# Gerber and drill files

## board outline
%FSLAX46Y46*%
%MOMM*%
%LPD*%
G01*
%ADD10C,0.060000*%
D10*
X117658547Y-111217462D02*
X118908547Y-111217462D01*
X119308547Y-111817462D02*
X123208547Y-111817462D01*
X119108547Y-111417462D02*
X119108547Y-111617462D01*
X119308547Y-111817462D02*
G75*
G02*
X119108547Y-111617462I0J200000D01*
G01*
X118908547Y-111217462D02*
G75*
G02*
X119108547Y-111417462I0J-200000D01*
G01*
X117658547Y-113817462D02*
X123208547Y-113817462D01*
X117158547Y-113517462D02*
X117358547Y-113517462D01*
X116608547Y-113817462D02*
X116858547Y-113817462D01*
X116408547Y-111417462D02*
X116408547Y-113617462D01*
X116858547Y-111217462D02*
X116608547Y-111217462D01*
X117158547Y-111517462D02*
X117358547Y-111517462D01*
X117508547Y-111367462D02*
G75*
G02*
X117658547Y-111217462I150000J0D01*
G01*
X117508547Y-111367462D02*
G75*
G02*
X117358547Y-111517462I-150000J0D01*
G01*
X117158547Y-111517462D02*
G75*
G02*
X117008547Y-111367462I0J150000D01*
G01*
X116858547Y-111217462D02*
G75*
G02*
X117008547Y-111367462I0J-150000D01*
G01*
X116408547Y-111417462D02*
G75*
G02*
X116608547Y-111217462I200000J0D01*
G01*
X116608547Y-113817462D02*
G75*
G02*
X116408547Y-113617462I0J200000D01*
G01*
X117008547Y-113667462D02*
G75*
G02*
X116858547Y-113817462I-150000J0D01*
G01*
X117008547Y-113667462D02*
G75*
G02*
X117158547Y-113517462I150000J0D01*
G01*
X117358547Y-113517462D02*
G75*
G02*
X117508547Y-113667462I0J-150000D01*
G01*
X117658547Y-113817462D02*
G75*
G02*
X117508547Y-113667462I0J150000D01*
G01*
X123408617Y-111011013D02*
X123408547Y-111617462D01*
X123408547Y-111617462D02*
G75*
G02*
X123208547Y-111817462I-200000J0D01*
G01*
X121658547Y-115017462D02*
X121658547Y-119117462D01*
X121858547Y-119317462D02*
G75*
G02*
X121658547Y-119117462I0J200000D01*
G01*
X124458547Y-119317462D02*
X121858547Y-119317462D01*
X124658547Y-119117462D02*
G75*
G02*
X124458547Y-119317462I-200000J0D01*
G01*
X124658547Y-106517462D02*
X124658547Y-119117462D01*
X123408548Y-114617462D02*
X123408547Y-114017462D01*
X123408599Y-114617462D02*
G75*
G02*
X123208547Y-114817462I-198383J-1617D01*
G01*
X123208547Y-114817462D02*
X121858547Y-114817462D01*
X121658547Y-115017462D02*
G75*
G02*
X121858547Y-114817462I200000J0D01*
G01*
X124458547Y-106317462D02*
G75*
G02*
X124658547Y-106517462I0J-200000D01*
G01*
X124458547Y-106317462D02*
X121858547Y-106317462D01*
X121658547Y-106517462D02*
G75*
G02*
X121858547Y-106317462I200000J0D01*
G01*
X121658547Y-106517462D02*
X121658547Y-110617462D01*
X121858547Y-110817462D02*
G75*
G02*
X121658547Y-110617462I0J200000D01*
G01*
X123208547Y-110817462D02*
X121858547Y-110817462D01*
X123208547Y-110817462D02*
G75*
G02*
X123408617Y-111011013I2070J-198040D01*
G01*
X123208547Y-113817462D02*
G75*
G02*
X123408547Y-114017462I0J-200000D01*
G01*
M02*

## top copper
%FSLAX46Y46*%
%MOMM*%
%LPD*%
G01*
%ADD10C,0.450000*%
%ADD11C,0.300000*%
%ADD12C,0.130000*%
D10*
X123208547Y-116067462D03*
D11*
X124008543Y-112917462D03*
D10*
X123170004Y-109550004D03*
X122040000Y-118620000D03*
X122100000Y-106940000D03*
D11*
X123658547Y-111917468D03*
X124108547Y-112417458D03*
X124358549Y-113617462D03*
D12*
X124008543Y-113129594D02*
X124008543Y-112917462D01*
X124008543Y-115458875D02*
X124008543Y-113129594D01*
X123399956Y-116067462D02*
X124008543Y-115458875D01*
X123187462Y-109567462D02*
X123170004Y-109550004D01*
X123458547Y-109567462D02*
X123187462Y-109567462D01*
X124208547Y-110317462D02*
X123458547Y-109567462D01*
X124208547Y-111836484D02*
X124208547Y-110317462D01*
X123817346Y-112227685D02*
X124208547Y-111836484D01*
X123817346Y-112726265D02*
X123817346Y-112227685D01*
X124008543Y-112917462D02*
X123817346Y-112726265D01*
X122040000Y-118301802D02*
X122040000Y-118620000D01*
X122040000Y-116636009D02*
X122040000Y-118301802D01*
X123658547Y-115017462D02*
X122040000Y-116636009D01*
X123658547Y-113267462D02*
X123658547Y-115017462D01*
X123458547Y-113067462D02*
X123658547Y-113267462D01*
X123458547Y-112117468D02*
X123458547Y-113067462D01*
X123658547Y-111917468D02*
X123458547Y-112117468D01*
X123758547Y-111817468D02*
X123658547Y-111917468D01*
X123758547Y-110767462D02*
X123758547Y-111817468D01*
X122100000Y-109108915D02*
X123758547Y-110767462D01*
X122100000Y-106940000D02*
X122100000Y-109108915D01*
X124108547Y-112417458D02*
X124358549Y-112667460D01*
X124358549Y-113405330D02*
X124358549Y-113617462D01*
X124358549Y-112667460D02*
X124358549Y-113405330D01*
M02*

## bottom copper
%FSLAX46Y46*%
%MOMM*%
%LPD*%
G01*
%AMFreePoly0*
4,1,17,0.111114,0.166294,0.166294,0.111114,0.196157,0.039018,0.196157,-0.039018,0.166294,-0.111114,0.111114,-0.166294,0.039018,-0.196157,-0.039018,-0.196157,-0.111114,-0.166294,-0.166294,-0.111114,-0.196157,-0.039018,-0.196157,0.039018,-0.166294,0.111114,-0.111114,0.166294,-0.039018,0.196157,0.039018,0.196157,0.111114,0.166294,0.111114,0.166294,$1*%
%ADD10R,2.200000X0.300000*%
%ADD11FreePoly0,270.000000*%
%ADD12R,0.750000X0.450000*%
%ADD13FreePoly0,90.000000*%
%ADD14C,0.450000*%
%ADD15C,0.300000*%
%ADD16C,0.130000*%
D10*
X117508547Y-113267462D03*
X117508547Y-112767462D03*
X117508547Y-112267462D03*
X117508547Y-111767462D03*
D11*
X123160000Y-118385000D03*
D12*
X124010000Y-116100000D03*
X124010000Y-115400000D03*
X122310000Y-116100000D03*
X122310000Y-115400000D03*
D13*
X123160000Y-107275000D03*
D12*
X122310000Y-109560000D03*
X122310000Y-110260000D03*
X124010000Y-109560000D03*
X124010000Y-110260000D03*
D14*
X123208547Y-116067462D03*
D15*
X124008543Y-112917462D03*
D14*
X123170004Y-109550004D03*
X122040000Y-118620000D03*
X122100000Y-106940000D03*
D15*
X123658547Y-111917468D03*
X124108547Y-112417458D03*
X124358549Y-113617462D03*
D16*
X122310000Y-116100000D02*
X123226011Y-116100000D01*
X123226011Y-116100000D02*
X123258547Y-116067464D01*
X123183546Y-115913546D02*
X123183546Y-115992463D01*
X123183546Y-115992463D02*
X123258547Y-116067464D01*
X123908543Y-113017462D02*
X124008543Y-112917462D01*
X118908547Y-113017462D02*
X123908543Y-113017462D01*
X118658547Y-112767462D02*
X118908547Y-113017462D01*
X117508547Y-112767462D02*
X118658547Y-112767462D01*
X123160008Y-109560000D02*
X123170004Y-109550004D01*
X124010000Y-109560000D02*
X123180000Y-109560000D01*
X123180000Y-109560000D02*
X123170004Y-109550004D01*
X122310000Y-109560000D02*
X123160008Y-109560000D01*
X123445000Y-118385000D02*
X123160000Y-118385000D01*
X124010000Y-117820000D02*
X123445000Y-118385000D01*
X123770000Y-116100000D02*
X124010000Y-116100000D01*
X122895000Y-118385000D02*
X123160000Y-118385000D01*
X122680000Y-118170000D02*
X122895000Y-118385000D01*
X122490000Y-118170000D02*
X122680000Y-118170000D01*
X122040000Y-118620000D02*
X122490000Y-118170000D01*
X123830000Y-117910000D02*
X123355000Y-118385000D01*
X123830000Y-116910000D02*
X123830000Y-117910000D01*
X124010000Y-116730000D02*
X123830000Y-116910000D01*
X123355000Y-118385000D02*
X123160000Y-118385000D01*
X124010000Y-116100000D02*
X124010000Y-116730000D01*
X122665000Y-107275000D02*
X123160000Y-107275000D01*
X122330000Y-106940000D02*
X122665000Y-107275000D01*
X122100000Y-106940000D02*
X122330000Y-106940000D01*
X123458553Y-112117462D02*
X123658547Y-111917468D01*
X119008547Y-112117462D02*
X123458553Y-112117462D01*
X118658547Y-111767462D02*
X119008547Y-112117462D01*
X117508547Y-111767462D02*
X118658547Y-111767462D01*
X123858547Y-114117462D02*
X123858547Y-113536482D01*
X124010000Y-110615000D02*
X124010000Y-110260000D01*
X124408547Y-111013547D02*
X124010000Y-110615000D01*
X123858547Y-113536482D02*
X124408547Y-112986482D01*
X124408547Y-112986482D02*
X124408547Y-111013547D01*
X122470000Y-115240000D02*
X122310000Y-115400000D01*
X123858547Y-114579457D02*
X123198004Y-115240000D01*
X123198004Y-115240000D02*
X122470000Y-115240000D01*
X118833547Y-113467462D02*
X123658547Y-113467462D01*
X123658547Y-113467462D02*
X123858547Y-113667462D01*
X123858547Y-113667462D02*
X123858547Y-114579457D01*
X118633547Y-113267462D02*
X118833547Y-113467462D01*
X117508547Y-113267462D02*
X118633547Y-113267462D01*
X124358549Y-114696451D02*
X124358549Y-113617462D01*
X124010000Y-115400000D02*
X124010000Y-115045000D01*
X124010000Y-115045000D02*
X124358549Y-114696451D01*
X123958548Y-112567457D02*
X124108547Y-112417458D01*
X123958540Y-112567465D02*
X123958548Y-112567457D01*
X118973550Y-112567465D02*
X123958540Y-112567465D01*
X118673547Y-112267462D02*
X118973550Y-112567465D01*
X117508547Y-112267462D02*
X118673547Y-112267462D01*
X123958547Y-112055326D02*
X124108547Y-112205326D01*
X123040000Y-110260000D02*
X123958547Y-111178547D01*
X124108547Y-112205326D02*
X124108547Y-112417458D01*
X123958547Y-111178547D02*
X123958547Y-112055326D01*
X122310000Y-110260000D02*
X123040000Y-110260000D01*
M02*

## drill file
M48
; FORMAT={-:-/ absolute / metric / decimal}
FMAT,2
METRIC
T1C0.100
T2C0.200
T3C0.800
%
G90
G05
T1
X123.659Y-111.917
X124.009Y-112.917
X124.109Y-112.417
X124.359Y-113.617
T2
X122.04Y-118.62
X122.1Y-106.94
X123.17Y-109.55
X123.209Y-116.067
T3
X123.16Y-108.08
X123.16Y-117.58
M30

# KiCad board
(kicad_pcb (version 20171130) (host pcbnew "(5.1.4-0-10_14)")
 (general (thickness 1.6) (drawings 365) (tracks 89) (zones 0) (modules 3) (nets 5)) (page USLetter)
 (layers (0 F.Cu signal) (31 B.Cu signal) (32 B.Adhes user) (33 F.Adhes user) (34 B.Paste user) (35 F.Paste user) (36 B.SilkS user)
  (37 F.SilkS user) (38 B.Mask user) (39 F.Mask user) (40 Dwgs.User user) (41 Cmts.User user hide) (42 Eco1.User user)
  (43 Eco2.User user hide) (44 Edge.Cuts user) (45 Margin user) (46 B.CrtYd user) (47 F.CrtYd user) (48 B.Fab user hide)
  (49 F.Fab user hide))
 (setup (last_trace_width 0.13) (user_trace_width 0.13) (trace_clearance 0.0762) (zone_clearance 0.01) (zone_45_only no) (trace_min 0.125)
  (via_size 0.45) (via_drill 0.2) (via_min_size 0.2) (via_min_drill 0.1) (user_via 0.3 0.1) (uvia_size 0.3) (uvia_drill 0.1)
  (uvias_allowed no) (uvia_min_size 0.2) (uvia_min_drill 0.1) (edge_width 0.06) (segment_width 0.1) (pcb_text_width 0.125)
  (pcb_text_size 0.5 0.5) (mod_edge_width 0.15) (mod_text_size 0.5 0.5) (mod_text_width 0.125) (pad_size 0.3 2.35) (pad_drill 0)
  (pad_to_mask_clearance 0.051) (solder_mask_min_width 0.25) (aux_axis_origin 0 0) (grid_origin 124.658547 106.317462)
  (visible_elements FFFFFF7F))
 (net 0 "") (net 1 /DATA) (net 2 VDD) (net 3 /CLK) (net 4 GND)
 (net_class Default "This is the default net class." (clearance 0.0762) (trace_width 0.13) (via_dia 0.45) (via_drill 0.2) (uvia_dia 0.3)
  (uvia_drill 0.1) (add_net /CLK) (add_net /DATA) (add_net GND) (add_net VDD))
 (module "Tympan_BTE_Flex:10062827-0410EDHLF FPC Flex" (layer B.Cu) (at 116.408547 111.217462 270)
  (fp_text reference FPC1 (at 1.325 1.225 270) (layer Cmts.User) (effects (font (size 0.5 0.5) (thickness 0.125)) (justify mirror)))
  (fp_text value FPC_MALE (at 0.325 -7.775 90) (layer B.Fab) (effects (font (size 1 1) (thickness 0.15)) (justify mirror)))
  (pad 1 smd rect (at 2.05 -1.1 270) (size 0.3 2.2) (layers B.Cu B.Mask) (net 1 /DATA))
  (pad 2 smd rect (at 1.55 -1.1 270) (size 0.3 2.2) (layers B.Cu B.Mask) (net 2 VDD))
  (pad 3 smd rect (at 1.05 -1.1 270) (size 0.3 2.2) (layers B.Cu B.Mask) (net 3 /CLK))
  (pad 4 smd rect (at 0.55 -1.1 270) (size 0.3 2.2) (layers B.Cu B.Mask) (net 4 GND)))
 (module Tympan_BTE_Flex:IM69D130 (layer B.Cu) (at 123.16 117.58 270)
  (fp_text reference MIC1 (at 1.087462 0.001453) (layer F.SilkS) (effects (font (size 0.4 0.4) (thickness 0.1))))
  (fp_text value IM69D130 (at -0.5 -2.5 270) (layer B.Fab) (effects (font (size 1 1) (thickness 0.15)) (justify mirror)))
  (pad "" np_thru_hole circle (at 0 0 270) (size 0.8 0.8) (drill 0.8) (layers *.Cu *.Mask))
  (pad 5 smd custom (at 0.805 0 270) (size 0.4 0.4) (layers B.Cu B.Mask) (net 4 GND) (zone_connect 0)
   (options (clearance outline) (anchor circle)) (primitives))
  (pad 4 smd rect (at -1.48 -0.85 270) (size 0.45 0.75) (layers B.Cu B.Mask) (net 4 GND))
  (pad 3 smd rect (at -2.18 -0.85 270) (size 0.45 0.75) (layers B.Cu B.Mask) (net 3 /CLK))
  (pad 2 smd rect (at -1.48 0.85 270) (size 0.45 0.75) (layers B.Cu B.Mask) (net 2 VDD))
  (pad 1 smd rect (at -2.18 0.85 270) (size 0.45 0.75) (layers B.Cu B.Mask) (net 1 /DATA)))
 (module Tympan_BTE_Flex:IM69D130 (layer B.Cu) (at 123.16 108.76 90)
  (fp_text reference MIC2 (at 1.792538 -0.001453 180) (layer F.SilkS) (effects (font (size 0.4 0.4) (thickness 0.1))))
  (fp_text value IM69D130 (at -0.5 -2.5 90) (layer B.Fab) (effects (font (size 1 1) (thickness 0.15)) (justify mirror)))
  (pad "" np_thru_hole circle (at 0.68 0 90) (size 0.8 0.8) (drill 0.8) (layers *.Cu *.Mask))
  (pad 5 smd custom (at 1.485 0 90) (size 0.4 0.4) (layers B.Cu B.Mask) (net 4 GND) (zone_connect 0)
   (options (clearance outline) (anchor circle)) (primitives))
  (pad 4 smd rect (at -0.8 -0.85 90) (size 0.45 0.75) (layers B.Cu B.Mask) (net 2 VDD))
  (pad 3 smd rect (at -1.5 -0.85 90) (size 0.45 0.75) (layers B.Cu B.Mask) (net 3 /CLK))
  (pad 2 smd rect (at -0.8 0.85 90) (size 0.45 0.75) (layers B.Cu B.Mask) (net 2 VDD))
  (pad 1 smd rect (at -1.5 0.85 90) (size 0.45 0.75) (layers B.Cu B.Mask) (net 1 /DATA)))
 (gr_line (start 117.658547 111.217462) (end 118.908547 111.217462) (layer Edge.Cuts) (width 0.06))
 (gr_line (start 119.308547 111.817462) (end 123.208547 111.817462) (layer Edge.Cuts) (width 0.06))
 (gr_line (start 119.108547 111.417462) (end 119.108547 111.617462) (layer Edge.Cuts) (width 0.06))
 (gr_arc (start 119.308547 111.617462) (end 119.108547 111.617462) (angle -90) (layer Edge.Cuts) (width 0.06))
 (gr_arc (start 118.908547 111.417462) (end 119.108547 111.417462) (angle -90) (layer Edge.Cuts) (width 0.06))
 (gr_line (start 117.658547 113.817462) (end 123.208547 113.817462) (layer Edge.Cuts) (width 0.06))
 (gr_line (start 117.158547 113.517462) (end 117.358547 113.517462) (layer Edge.Cuts) (width 0.06))
 (gr_line (start 116.608547 113.817462) (end 116.858547 113.817462) (layer Edge.Cuts) (width 0.06))
 (gr_line (start 116.408547 111.417462) (end 116.408547 113.617462) (layer Edge.Cuts) (width 0.06))
 (gr_line (start 116.858547 111.217462) (end 116.608547 111.217462) (layer Edge.Cuts) (width 0.06))
 (gr_line (start 117.158547 111.517462) (end 117.358547 111.517462) (layer Edge.Cuts) (width 0.06))
 (gr_arc (start 117.658547 111.367462) (end 117.658547 111.217462) (angle -90) (layer Edge.Cuts) (width 0.06))
 (gr_arc (start 117.358547 111.367462) (end 117.358547 111.517462) (angle -90) (layer Edge.Cuts) (width 0.06))
 (gr_arc (start 117.158547 111.367462) (end 117.008547 111.367462) (angle -90) (layer Edge.Cuts) (width 0.06))
 (gr_arc (start 116.858547 111.367462) (end 117.008547 111.367462) (angle -90) (layer Edge.Cuts) (width 0.06))
 (gr_arc (start 116.608547 111.417462) (end 116.608547 111.217462) (angle -90) (layer Edge.Cuts) (width 0.06))
 (gr_arc (start 116.608547 113.617462) (end 116.408547 113.617462) (angle -90) (layer Edge.Cuts) (width 0.06))
 (gr_arc (start 116.858547 113.667462) (end 116.858547 113.817462) (angle -90) (layer Edge.Cuts) (width 0.06))
 (gr_arc (start 117.158547 113.667462) (end 117.158547 113.517462) (angle -90) (layer Edge.Cuts) (width 0.06))
 (gr_arc (start 117.358547 113.667462) (end 117.508547 113.667462) (angle -90) (layer Edge.Cuts) (width 0.06))
 (gr_arc (start 117.658547 113.667462) (end 117.508547 113.667462) (angle -90) (layer Edge.Cuts) (width 0.06))
 (gr_line (start 123.408617 111.011013) (end 123.408547 111.617462) (layer Edge.Cuts) (width 0.06))
 (gr_arc (start 123.208547 111.617462) (end 123.208547 111.817462) (angle -90) (layer Edge.Cuts) (width 0.06))
 (gr_line (start 121.658547 115.017462) (end 121.658547 119.117462) (layer Edge.Cuts) (width 0.06))
 (gr_arc (start 121.858547 119.117462) (end 121.658547 119.117462) (angle -90) (layer Edge.Cuts) (width 0.06))
 (gr_line (start 124.458547 119.317462) (end 121.858547 119.317462) (layer Edge.Cuts) (width 0.06))
 (gr_arc (start 124.458547 119.117462) (end 124.458547 119.317462) (angle -90) (layer Edge.Cuts) (width 0.06))
 (gr_line (start 124.658547 106.517462) (end 124.658547 119.117462) (layer Edge.Cuts) (width 0.06))
 (gr_line (start 123.408548 114.617462) (end 123.408547 114.017462) (layer Edge.Cuts) (width 0.06))
 (gr_arc (start 123.210216 114.619079) (end 123.208547 114.817462) (angle -90.94914104) (layer Edge.Cuts) (width 0.06))
 (gr_line (start 123.208547 114.817462) (end 121.858547 114.817462) (layer Edge.Cuts) (width 0.06))
 (gr_arc (start 121.858547 115.017462) (end 121.858547 114.817462) (angle -90) (layer Edge.Cuts) (width 0.06))
 (gr_arc (start 124.458547 106.517462) (end 124.658547 106.517462) (angle -90) (layer Edge.Cuts) (width 0.06))
 (gr_line (start 124.458547 106.317462) (end 121.858547 106.317462) (layer Edge.Cuts) (width 0.06))
 (gr_arc (start 121.858547 106.517462) (end 121.858547 106.317462) (angle -90) (layer Edge.Cuts) (width 0.06))
 (gr_line (start 121.658547 106.517462) (end 121.658547 110.617462) (layer Edge.Cuts) (width 0.06))
 (gr_arc (start 121.858547 110.617462) (end 121.658547 110.617462) (angle -90) (layer Edge.Cuts) (width 0.06))
 (gr_line (start 123.208547 110.817462) (end 121.858547 110.817462) (layer Edge.Cuts) (width 0.06))
 (gr_arc (start 123.210617 111.015502) (end 123.408617 111.011013) (angle -89.3) (layer Edge.Cuts) (width 0.06))
 (gr_arc (start 123.208547 114.017462) (end 123.408547 114.017462) (angle -90) (layer Edge.Cuts) (width 0.06))
 (via (at 123.208547 116.067462) (size 0.45) (drill 0.2) (layers F.Cu B.Cu) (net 2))
 (segment (start 122.31 116.1) (end 123.226011 116.1) (width 0.13) (layer B.Cu) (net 2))
 (segment (start 123.226011 116.1) (end 123.258547 116.067464) (width 0.13) (layer B.Cu) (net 2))
 (segment (start 123.183546 115.913546) (end 123.183546 115.992463) (width 0.13) (layer B.Cu) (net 2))
 (segment (start 123.183546 115.992463) (end 123.258547 116.067464) (width 0.13) (layer B.Cu) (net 2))
 (via (at 124.008543 112.917462) (size 0.3) (drill 0.1) (layers F.Cu B.Cu) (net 2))
 (segment (start 124.008543 113.129594) (end 124.008543 112.917462) (width 0.13) (layer F.Cu) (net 2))
 (segment (start 124.008543 115.458875) (end 124.008543 113.129594) (width 0.13) (layer F.Cu) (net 2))
 (segment (start 123.399956 116.067462) (end 124.008543 115.458875) (width 0.13) (layer F.Cu) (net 2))
 (segment (start 123.908543 113.017462) (end 124.008543 112.917462) (width 0.13) (layer B.Cu) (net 2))
 (segment (start 118.908547 113.017462) (end 123.908543 113.017462) (width 0.13) (layer B.Cu) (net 2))
 (segment (start 118.658547 112.767462) (end 118.908547 113.017462) (width 0.13) (layer B.Cu) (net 2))
 (segment (start 117.508547 112.767462) (end 118.658547 112.767462) (width 0.13) (layer B.Cu) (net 2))
 (via (at 123.170004 109.550004) (size 0.45) (drill 0.2) (layers F.Cu B.Cu) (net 2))
 (segment (start 123.160008 109.56) (end 123.170004 109.550004) (width 0.13) (layer B.Cu) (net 2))
 (segment (start 124.01 109.56) (end 123.18 109.56) (width 0.13) (layer B.Cu) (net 2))
 (segment (start 123.18 109.56) (end 123.170004 109.550004) (width 0.13) (layer B.Cu) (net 2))
 (segment (start 122.31 109.56) (end 123.160008 109.56) (width 0.13) (layer B.Cu) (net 2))
 (segment (start 123.187462 109.567462) (end 123.170004 109.550004) (width 0.13) (layer F.Cu) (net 2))
 (segment (start 123.458547 109.567462) (end 123.187462 109.567462) (width 0.13) (layer F.Cu) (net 2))
 (segment (start 124.208547 110.317462) (end 123.458547 109.567462) (width 0.13) (layer F.Cu) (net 2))
 (segment (start 124.208547 111.836484) (end 124.208547 110.317462) (width 0.13) (layer F.Cu) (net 2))
 (segment (start 123.817346 112.227685) (end 124.208547 111.836484) (width 0.13) (layer F.Cu) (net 2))
 (segment (start 123.817346 112.726265) (end 123.817346 112.227685) (width 0.13) (layer F.Cu) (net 2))
 (segment (start 124.008543 112.917462) (end 123.817346 112.726265) (width 0.13) (layer F.Cu) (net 2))
 (segment (start 123.445 118.385) (end 123.16 118.385) (width 0.13) (layer B.Cu) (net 4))
 (segment (start 124.01 117.82) (end 123.445 118.385) (width 0.13) (layer B.Cu) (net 4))
 (segment (start 123.77 116.1) (end 124.01 116.1) (width 0.13) (layer B.Cu) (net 4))
 (via (at 122.04 118.62) (size 0.45) (drill 0.2) (layers F.Cu B.Cu) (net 4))
 (segment (start 122.895 118.385) (end 123.16 118.385) (width 0.13) (layer B.Cu) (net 4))
 (segment (start 122.68 118.17) (end 122.895 118.385) (width 0.13) (layer B.Cu) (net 4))
 (segment (start 122.49 118.17) (end 122.68 118.17) (width 0.13) (layer B.Cu) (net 4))
 (segment (start 122.04 118.62) (end 122.49 118.17) (width 0.13) (layer B.Cu) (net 4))
 (segment (start 123.83 117.91) (end 123.355 118.385) (width 0.13) (layer B.Cu) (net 4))
 (segment (start 123.83 116.91) (end 123.83 117.91) (width 0.13) (layer B.Cu) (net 4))
 (segment (start 124.01 116.73) (end 123.83 116.91) (width 0.13) (layer B.Cu) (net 4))
 (segment (start 123.355 118.385) (end 123.16 118.385) (width 0.13) (layer B.Cu) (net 4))
 (segment (start 124.01 116.1) (end 124.01 116.73) (width 0.13) (layer B.Cu) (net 4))
 (via (at 122.1 106.94) (size 0.45) (drill 0.2) (layers F.Cu B.Cu) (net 4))
 (segment (start 122.665 107.275) (end 123.16 107.275) (width 0.13) (layer B.Cu) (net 4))
 (segment (start 122.33 106.94) (end 122.665 107.275) (width 0.13) (layer B.Cu) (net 4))
 (segment (start 122.1 106.94) (end 122.33 106.94) (width 0.13) (layer B.Cu) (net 4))
 (via (at 123.658547 111.917468) (size 0.3) (drill 0.1) (layers F.Cu B.Cu) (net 4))
 (segment (start 123.458553 112.117462) (end 123.658547 111.917468) (width 0.13) (layer B.Cu) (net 4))
 (segment (start 119.008547 112.117462) (end 123.458553 112.117462) (width 0.13) (layer B.Cu) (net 4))
 (segment (start 118.658547 111.767462) (end 119.008547 112.117462) (width 0.13) (layer B.Cu) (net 4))
 (segment (start 117.508547 111.767462) (end 118.658547 111.767462) (width 0.13) (layer B.Cu) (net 4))
 (segment (start 122.04 118.301802) (end 122.04 118.62) (width 0.13) (layer F.Cu) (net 4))
 (segment (start 122.04 116.636009) (end 122.04 118.301802) (width 0.13) (layer F.Cu) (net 4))
 (segment (start 123.658547 115.017462) (end 122.04 116.636009) (width 0.13) (layer F.Cu) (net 4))
 (segment (start 123.658547 113.267462) (end 123.658547 115.017462) (width 0.13) (layer F.Cu) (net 4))
 (segment (start 123.458547 113.067462) (end 123.658547 113.267462) (width 0.13) (layer F.Cu) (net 4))
 (segment (start 123.458547 112.117468) (end 123.458547 113.067462) (width 0.13) (layer F.Cu) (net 4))
 (segment (start 123.658547 111.917468) (end 123.458547 112.117468) (width 0.13) (layer F.Cu) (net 4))
 (segment (start 123.758547 111.817468) (end 123.658547 111.917468) (width 0.13) (layer F.Cu) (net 4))
 (segment (start 123.758547 110.767462) (end 123.758547 111.817468) (width 0.13) (layer F.Cu) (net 4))
 (segment (start 122.1 109.108915) (end 123.758547 110.767462) (width 0.13) (layer F.Cu) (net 4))
 (segment (start 122.1 106.94) (end 122.1 109.108915) (width 0.13) (layer F.Cu) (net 4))
 (segment (start 123.858547 114.117462) (end 123.858547 113.536482) (width 0.13) (layer B.Cu) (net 1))
 (segment (start 124.01 110.615) (end 124.01 110.26) (width 0.13) (layer B.Cu) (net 1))
 (segment (start 124.408547 111.013547) (end 124.01 110.615) (width 0.13) (layer B.Cu) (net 1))
 (segment (start 123.858547 113.536482) (end 124.408547 112.986482) (width 0.13) (layer B.Cu) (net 1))
 (segment (start 124.408547 112.986482) (end 124.408547 111.013547) (width 0.13) (layer B.Cu) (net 1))
 (segment (start 122.47 115.24) (end 122.31 115.4) (width 0.13) (layer B.Cu) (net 1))
 (segment (start 123.858547 114.579457) (end 123.198004 115.24) (width 0.13) (layer B.Cu) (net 1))
 (segment (start 123.198004 115.24) (end 122.47 115.24) (width 0.13) (layer B.Cu) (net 1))
 (segment (start 118.833547 113.467462) (end 123.658547 113.467462) (width 0.13) (layer B.Cu) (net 1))
 (segment (start 123.658547 113.467462) (end 123.858547 113.667462) (width 0.13) (layer B.Cu) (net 1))
 (segment (start 123.858547 113.667462) (end 123.858547 114.579457) (width 0.13) (layer B.Cu) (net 1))
 (segment (start 118.633547 113.267462) (end 118.833547 113.467462) (width 0.13) (layer B.Cu) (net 1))
 (segment (start 117.508547 113.267462) (end 118.633547 113.267462) (width 0.13) (layer B.Cu) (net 1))
 (via (at 124.108547 112.417458) (size 0.3) (drill 0.1) (layers F.Cu B.Cu) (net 3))
 (via (at 124.358549 113.617462) (size 0.3) (drill 0.1) (layers F.Cu B.Cu) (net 3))
 (segment (start 124.358549 114.696451) (end 124.358549 113.617462) (width 0.13) (layer B.Cu) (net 3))
 (segment (start 124.108547 112.417458) (end 124.358549 112.66746) (width 0.13) (layer F.Cu) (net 3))
 (segment (start 124.358549 113.40533) (end 124.358549 113.617462) (width 0.13) (layer F.Cu) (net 3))
 (segment (start 124.358549 112.66746) (end 124.358549 113.40533) (width 0.13) (layer F.Cu) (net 3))
 (segment (start 124.01 115.4) (end 124.01 115.045) (width 0.13) (layer B.Cu) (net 3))
 (segment (start 124.01 115.045) (end 124.358549 114.696451) (width 0.13) (layer B.Cu) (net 3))
 (segment (start 123.958548 112.567457) (end 124.108547 112.417458) (width 0.13) (layer B.Cu) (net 3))
 (segment (start 123.95854 112.567465) (end 123.958548 112.567457) (width 0.13) (layer B.Cu) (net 3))
 (segment (start 118.97355 112.567465) (end 123.95854 112.567465) (width 0.13) (layer B.Cu) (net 3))
 (segment (start 118.673547 112.267462) (end 118.97355 112.567465) (width 0.13) (layer B.Cu) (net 3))
 (segment (start 117.508547 112.267462) (end 118.673547 112.267462) (width 0.13) (layer B.Cu) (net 3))
 (segment (start 123.958547 112.055326) (end 124.108547 112.205326) (width 0.13) (layer B.Cu) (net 3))
 (segment (start 123.04 110.26) (end 123.958547 111.178547) (width 0.13) (layer B.Cu) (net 3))
 (segment (start 124.108547 112.205326) (end 124.108547 112.417458) (width 0.13) (layer B.Cu) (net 3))
 (segment (start 123.958547 111.178547) (end 123.958547 112.055326) (width 0.13) (layer B.Cu) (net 3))
 (segment (start 122.31 110.26) (end 123.04 110.26) (width 0.13) (layer B.Cu) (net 3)))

